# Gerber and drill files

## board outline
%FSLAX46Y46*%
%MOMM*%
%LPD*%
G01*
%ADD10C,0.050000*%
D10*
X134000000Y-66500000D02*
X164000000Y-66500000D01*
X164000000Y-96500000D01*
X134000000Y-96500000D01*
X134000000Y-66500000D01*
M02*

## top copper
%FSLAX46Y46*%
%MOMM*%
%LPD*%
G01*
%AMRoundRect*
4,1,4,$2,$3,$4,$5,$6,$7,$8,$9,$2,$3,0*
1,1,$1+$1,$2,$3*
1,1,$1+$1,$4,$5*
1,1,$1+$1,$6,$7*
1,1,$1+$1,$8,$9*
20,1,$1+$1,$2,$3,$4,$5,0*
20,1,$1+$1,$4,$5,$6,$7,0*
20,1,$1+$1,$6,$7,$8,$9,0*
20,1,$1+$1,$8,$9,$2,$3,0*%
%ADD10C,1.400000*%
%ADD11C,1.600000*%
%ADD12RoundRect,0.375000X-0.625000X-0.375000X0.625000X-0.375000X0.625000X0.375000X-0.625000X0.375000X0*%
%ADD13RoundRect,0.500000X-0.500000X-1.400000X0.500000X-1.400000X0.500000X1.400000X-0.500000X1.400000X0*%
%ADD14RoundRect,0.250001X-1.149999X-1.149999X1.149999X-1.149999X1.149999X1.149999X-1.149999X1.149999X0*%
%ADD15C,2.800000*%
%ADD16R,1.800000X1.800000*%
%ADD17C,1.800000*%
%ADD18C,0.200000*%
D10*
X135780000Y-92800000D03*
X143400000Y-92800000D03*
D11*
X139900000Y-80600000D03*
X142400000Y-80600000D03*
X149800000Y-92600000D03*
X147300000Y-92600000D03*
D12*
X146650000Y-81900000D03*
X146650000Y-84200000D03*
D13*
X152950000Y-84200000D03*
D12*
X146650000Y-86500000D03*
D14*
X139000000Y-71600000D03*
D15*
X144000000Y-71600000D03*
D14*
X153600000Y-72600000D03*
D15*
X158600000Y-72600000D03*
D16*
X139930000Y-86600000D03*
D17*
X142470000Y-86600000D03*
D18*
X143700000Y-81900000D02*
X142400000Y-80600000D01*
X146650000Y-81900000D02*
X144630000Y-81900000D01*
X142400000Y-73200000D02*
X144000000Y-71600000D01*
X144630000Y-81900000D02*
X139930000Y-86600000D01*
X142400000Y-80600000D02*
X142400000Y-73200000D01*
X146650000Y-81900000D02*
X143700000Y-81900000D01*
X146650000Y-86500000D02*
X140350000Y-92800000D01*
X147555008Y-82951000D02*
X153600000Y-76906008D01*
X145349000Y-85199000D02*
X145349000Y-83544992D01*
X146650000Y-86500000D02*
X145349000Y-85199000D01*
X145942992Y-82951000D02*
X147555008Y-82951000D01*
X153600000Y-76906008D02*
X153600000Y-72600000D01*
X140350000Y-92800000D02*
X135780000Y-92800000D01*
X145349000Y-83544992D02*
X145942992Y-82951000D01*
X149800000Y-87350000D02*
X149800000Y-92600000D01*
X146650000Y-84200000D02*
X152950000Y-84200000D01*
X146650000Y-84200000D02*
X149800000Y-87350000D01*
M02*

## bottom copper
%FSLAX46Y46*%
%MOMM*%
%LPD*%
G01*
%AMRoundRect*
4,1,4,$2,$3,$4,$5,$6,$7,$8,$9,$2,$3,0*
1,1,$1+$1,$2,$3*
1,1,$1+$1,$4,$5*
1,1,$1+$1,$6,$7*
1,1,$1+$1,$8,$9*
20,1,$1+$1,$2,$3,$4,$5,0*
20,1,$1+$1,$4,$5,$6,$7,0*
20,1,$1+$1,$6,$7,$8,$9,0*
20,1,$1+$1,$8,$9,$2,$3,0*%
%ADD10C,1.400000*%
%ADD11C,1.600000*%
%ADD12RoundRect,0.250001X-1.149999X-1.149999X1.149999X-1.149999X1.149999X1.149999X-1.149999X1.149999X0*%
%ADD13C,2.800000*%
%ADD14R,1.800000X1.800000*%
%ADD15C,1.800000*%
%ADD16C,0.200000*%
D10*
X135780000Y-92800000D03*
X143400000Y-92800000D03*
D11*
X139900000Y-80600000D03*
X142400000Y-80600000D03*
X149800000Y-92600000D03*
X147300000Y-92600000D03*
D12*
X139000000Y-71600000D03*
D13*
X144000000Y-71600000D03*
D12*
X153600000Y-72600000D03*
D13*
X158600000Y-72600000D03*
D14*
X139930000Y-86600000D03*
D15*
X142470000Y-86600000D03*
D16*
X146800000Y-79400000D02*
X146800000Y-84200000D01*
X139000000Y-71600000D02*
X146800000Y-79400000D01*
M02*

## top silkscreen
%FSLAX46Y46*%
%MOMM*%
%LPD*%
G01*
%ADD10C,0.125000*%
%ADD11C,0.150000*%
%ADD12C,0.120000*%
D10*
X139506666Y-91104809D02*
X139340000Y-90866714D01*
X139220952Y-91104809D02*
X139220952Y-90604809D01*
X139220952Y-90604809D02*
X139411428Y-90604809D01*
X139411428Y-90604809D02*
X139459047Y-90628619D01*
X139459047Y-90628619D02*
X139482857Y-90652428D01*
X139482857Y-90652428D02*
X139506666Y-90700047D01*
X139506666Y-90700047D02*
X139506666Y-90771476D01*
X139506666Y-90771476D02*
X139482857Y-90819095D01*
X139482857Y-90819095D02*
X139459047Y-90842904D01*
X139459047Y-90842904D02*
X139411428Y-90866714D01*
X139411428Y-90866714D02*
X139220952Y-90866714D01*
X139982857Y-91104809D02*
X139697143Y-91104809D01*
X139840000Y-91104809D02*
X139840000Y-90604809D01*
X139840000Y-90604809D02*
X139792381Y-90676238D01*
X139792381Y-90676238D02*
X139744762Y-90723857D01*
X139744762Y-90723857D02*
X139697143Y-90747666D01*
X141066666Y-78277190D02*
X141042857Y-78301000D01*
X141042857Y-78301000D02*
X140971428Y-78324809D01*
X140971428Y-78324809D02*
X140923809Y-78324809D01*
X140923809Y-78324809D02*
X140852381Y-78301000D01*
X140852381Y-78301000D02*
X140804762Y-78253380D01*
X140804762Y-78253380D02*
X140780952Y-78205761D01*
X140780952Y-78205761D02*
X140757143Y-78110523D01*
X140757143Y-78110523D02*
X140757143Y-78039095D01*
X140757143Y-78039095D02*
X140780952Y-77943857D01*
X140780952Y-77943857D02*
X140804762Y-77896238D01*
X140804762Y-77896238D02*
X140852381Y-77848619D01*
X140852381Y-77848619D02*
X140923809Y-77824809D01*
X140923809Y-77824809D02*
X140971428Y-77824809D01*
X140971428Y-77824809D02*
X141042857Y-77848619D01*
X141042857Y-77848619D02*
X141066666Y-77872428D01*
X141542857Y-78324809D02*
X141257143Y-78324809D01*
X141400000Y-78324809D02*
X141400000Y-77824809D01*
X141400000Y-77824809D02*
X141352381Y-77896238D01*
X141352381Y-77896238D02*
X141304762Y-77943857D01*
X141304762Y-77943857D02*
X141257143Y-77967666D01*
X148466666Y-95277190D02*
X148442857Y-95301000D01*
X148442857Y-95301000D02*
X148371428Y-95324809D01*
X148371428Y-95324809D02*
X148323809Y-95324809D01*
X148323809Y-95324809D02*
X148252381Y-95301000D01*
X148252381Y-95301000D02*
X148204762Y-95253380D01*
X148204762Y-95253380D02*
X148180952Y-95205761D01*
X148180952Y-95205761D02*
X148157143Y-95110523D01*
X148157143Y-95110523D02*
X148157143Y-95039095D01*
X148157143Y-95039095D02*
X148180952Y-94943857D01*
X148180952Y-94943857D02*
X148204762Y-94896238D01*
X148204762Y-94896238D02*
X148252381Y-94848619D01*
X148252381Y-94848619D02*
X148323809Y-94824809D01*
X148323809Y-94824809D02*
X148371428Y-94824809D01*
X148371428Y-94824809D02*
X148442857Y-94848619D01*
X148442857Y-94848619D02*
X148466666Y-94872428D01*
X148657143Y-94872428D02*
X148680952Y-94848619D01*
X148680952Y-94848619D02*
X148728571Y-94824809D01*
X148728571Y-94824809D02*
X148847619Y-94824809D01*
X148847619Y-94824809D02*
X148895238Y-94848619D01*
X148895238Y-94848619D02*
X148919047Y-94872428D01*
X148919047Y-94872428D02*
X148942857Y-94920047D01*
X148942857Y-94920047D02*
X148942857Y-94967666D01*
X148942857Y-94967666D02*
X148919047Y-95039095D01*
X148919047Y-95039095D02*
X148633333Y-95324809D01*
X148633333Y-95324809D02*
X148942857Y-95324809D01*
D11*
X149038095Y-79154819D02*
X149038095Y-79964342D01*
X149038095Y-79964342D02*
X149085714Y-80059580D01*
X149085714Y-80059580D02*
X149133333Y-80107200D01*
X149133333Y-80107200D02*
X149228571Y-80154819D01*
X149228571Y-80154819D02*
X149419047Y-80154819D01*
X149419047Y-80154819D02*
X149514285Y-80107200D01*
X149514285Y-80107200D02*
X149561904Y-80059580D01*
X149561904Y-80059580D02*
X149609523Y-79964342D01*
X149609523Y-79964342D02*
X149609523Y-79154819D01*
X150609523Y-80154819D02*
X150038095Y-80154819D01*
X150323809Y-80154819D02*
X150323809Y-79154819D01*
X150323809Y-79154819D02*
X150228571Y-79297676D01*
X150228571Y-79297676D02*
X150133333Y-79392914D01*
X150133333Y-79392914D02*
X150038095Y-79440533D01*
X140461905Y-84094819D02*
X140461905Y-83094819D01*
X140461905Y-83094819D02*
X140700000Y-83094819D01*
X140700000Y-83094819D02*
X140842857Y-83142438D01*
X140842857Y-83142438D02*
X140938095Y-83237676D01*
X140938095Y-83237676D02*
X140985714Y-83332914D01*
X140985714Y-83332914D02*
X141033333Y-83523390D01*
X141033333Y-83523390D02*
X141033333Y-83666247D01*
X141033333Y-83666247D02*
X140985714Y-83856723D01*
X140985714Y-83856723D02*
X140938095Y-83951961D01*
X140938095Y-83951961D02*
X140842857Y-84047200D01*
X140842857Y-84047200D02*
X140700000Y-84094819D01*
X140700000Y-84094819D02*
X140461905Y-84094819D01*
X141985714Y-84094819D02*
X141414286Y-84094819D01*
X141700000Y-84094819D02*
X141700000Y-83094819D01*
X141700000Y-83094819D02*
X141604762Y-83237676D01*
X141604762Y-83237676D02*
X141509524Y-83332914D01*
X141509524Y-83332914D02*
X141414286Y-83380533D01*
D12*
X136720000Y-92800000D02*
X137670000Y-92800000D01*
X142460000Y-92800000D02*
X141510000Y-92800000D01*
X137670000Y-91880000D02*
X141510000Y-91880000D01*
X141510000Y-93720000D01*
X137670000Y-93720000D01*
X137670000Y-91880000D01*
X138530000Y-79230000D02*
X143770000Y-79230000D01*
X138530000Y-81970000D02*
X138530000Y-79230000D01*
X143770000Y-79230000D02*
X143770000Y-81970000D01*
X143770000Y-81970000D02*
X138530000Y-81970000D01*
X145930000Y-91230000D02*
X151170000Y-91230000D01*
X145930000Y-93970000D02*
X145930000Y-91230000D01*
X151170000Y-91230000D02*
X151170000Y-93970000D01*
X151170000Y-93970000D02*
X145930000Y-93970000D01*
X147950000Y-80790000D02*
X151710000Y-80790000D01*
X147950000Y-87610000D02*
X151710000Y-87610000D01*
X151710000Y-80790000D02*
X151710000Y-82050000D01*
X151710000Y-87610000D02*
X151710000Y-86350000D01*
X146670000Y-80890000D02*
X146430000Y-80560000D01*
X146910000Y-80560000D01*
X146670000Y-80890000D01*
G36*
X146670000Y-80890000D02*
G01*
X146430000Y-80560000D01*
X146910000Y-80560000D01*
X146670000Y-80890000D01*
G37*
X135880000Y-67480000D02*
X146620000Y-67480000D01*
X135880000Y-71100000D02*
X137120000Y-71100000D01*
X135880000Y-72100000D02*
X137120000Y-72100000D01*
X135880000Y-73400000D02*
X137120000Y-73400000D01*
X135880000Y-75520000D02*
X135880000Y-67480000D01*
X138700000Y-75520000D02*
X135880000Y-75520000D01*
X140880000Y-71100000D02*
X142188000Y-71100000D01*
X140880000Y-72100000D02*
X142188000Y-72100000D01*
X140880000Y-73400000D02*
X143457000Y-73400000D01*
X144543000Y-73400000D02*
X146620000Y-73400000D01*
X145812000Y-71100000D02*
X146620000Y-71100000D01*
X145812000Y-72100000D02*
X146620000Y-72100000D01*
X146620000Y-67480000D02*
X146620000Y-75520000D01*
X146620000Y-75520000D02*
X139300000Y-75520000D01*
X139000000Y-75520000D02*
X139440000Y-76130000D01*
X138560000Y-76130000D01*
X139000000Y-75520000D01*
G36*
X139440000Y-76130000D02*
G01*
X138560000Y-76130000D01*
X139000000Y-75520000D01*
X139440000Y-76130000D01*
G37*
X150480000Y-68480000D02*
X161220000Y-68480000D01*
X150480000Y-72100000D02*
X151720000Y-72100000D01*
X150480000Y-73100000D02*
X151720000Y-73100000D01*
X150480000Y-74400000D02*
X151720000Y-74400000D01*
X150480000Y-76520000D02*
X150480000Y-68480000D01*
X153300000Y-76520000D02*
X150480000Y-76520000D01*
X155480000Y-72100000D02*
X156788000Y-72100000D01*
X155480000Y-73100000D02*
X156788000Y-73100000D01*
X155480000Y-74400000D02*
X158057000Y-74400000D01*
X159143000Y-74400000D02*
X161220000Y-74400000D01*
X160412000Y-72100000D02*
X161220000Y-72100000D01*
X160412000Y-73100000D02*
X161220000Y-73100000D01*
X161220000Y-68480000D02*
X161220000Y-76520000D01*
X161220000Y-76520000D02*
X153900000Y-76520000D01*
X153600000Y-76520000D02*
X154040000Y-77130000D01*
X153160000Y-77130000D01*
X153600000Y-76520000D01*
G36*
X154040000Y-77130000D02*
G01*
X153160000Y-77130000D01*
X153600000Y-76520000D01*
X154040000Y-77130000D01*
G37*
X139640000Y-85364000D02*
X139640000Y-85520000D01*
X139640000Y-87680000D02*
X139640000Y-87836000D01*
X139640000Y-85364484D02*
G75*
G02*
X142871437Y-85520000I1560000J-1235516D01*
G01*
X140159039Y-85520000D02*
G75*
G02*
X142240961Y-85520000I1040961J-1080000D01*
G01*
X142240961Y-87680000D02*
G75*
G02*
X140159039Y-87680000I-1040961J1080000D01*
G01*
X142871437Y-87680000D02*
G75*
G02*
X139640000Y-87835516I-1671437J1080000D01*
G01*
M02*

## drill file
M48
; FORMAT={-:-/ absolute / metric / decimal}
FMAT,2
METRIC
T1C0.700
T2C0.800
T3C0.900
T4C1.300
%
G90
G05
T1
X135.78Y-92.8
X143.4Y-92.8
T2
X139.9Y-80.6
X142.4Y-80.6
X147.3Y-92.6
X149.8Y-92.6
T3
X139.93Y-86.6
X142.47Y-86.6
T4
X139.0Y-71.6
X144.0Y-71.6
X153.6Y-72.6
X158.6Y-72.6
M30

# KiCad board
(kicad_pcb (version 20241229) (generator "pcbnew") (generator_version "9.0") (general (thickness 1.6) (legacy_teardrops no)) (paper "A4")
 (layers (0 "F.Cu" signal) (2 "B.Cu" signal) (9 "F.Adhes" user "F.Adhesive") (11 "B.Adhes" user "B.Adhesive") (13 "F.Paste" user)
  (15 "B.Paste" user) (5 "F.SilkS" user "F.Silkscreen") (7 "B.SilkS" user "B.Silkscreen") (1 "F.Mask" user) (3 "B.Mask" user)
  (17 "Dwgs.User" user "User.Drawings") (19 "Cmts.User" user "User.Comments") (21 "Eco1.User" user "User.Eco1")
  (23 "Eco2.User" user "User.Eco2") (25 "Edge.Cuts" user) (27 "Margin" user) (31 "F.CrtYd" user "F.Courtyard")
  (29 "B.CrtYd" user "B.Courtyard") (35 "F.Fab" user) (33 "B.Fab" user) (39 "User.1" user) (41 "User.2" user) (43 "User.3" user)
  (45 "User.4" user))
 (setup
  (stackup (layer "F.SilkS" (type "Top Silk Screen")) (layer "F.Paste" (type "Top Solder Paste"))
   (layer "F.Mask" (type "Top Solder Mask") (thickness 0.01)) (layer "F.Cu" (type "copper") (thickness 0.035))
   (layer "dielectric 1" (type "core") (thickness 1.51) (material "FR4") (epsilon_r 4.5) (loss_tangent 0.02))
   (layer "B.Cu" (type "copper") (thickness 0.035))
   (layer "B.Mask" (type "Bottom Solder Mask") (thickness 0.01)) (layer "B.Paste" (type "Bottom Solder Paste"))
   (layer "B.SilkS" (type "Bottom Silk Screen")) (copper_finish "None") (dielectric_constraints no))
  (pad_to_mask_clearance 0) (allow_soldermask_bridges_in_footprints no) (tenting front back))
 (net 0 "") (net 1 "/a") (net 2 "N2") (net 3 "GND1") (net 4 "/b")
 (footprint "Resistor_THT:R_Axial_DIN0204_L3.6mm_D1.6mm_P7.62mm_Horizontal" (layer "F.Cu") (at 135.78 92.8)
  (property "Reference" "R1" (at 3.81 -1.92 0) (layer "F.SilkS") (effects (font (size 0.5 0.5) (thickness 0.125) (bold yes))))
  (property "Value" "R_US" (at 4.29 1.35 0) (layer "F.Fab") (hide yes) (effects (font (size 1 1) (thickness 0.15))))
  (fp_line (start 0.94 0) (end 1.89 0) (stroke (width 0.12) (type solid)) (layer "F.SilkS"))
  (fp_line (start 6.68 0) (end 5.73 0) (stroke (width 0.12) (type solid)) (layer "F.SilkS"))
  (fp_rect (start 1.89 -0.92) (end 5.73 0.92) (stroke (width 0.12) (type solid)) (fill no) (layer "F.SilkS"))
  (pad "1" thru_hole circle (at 0 0) (size 1.4 1.4) (drill 0.7) (layers "*.Cu" "*.Mask") (remove_unused_layers no) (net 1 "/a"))
  (pad "2" thru_hole circle (at 7.62 0) (size 1.4 1.4) (drill 0.7) (layers "*.Cu" "*.Mask") (remove_unused_layers no) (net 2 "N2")))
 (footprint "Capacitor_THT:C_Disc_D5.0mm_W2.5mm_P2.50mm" (layer "F.Cu") (at 139.9 80.6)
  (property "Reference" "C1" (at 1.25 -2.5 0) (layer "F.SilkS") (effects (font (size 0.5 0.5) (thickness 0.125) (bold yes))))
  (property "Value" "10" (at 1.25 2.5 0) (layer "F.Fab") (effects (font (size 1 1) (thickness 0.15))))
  (fp_line (start -1.37 -1.37) (end 3.87 -1.37) (stroke (width 0.12) (type solid)) (layer "F.SilkS"))
  (fp_line (start -1.37 1.37) (end -1.37 -1.37) (stroke (width 0.12) (type solid)) (layer "F.SilkS"))
  (fp_line (start 3.87 -1.37) (end 3.87 1.37) (stroke (width 0.12) (type solid)) (layer "F.SilkS"))
  (fp_line (start 3.87 1.37) (end -1.37 1.37) (stroke (width 0.12) (type solid)) (layer "F.SilkS"))
  (pad "1" thru_hole circle (at 0 0) (size 1.6 1.6) (drill 0.8) (layers "*.Cu" "*.Mask") (remove_unused_layers no) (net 1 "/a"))
  (pad "2" thru_hole circle (at 2.5 0) (size 1.6 1.6) (drill 0.8) (layers "*.Cu" "*.Mask") (remove_unused_layers no) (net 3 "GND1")))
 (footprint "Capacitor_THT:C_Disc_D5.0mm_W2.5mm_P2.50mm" (layer "F.Cu") (at 149.8 92.6 180)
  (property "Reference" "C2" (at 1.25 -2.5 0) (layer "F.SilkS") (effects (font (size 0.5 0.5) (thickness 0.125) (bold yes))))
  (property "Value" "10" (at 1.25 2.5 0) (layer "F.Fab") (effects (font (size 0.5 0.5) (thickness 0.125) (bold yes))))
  (fp_line (start 3.87 1.37) (end -1.37 1.37) (stroke (width 0.12) (type solid)) (layer "F.SilkS"))
  (fp_line (start 3.87 -1.37) (end 3.87 1.37) (stroke (width 0.12) (type solid)) (layer "F.SilkS"))
  (fp_line (start -1.37 1.37) (end -1.37 -1.37) (stroke (width 0.12) (type solid)) (layer "F.SilkS"))
  (fp_line (start -1.37 -1.37) (end 3.87 -1.37) (stroke (width 0.12) (type solid)) (layer "F.SilkS"))
  (pad "1" thru_hole circle (at 0 0 180) (size 1.6 1.6) (drill 0.8) (layers "*.Cu" "*.Mask") (remove_unused_layers no) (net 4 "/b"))
  (pad "2" thru_hole circle (at 2.5 0 180) (size 1.6 1.6) (drill 0.8) (layers "*.Cu" "*.Mask") (remove_unused_layers no) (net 3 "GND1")))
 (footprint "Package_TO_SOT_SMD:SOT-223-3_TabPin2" (layer "F.Cu") (at 149.8 84.2)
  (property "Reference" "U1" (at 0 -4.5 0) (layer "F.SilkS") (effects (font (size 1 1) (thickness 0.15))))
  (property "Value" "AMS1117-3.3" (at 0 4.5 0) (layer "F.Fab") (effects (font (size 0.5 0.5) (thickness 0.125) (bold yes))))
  (fp_line (start -1.85 -3.41) (end 1.91 -3.41) (stroke (width 0.12) (type solid)) (layer "F.SilkS"))
  (fp_line (start -1.85 3.41) (end 1.91 3.41) (stroke (width 0.12) (type solid)) (layer "F.SilkS"))
  (fp_line (start 1.91 -3.41) (end 1.91 -2.15) (stroke (width 0.12) (type solid)) (layer "F.SilkS"))
  (fp_line (start 1.91 3.41) (end 1.91 2.15) (stroke (width 0.12) (type solid)) (layer "F.SilkS"))
  (fp_poly
   (pts (xy -3.13 -3.31) (xy -3.37 -3.64) (xy -2.89 -3.64) (xy -3.13 -3.31)) (stroke (width 0.12) (type solid)) (fill yes) (layer "F.SilkS"))
  (pad "1" smd roundrect (at -3.15 -2.3) (size 2 1.5) (layers "F.Cu" "F.Mask" "F.Paste") (roundrect_rratio 0.25) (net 3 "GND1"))
  (pad "2" smd roundrect (at -3.15 0) (size 2 1.5) (layers "F.Cu" "F.Mask" "F.Paste") (roundrect_rratio 0.25) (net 4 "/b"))
  (pad "2" smd roundrect (at 3.15 0) (size 2 3.8) (layers "F.Cu" "F.Mask" "F.Paste") (roundrect_rratio 0.25) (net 4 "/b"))
  (pad "3" smd roundrect (at -3.15 2.3) (size 2 1.5) (layers "F.Cu" "F.Mask" "F.Paste") (roundrect_rratio 0.25) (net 1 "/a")))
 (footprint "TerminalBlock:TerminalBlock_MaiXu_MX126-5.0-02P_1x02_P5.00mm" (layer "F.Cu") (at 139 71.6)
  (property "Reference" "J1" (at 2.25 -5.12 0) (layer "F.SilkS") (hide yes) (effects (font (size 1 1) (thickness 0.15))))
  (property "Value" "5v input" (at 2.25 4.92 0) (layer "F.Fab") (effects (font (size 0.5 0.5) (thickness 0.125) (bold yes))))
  (fp_line (start -3.12 -4.12) (end 7.62 -4.12) (stroke (width 0.12) (type solid)) (layer "F.SilkS"))
  (fp_line (start -3.12 -0.5) (end -1.88 -0.5) (stroke (width 0.12) (type solid)) (layer "F.SilkS"))
  (fp_line (start -3.12 0.5) (end -1.88 0.5) (stroke (width 0.12) (type solid)) (layer "F.SilkS"))
  (fp_line (start -3.12 1.8) (end -1.88 1.8) (stroke (width 0.12) (type solid)) (layer "F.SilkS"))
  (fp_line (start -3.12 3.92) (end -3.12 -4.12) (stroke (width 0.12) (type solid)) (layer "F.SilkS"))
  (fp_line (start -0.3 3.92) (end -3.12 3.92) (stroke (width 0.12) (type solid)) (layer "F.SilkS"))
  (fp_line (start 1.88 -0.5) (end 3.188 -0.5) (stroke (width 0.12) (type solid)) (layer "F.SilkS"))
  (fp_line (start 1.88 0.5) (end 3.188 0.5) (stroke (width 0.12) (type solid)) (layer "F.SilkS"))
  (fp_line (start 1.88 1.8) (end 4.457 1.8) (stroke (width 0.12) (type solid)) (layer "F.SilkS"))
  (fp_line (start 5.543 1.8) (end 7.62 1.8) (stroke (width 0.12) (type solid)) (layer "F.SilkS"))
  (fp_line (start 6.812 -0.5) (end 7.62 -0.5) (stroke (width 0.12) (type solid)) (layer "F.SilkS"))
  (fp_line (start 6.812 0.5) (end 7.62 0.5) (stroke (width 0.12) (type solid)) (layer "F.SilkS"))
  (fp_line (start 7.62 -4.12) (end 7.62 3.92) (stroke (width 0.12) (type solid)) (layer "F.SilkS"))
  (fp_line (start 7.62 3.92) (end 0.3 3.92) (stroke (width 0.12) (type solid)) (layer "F.SilkS"))
  (fp_poly (pts (xy 0 3.92) (xy 0.44 4.53) (xy -0.44 4.53)) (stroke (width 0.12) (type solid)) (fill yes) (layer "F.SilkS"))
  (pad "1" thru_hole roundrect (at 0 0) (size 2.8 2.8) (drill 1.3) (layers "*.Cu" "*.Mask") (remove_unused_layers no)
   (roundrect_rratio 0.089286) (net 4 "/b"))
  (pad "2" thru_hole circle (at 5 0) (size 2.8 2.8) (drill 1.3) (layers "*.Cu" "*.Mask") (remove_unused_layers no) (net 3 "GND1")))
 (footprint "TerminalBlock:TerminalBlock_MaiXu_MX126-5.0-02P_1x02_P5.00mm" (layer "F.Cu") (at 153.6 72.6)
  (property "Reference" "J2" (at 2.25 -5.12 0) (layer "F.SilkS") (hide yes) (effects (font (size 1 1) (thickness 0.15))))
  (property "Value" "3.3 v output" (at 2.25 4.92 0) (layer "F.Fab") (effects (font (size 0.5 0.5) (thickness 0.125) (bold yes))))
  (fp_line (start -3.12 -4.12) (end 7.62 -4.12) (stroke (width 0.12) (type solid)) (layer "F.SilkS"))
  (fp_line (start -3.12 -0.5) (end -1.88 -0.5) (stroke (width 0.12) (type solid)) (layer "F.SilkS"))
  (fp_line (start -3.12 0.5) (end -1.88 0.5) (stroke (width 0.12) (type solid)) (layer "F.SilkS"))
  (fp_line (start -3.12 1.8) (end -1.88 1.8) (stroke (width 0.12) (type solid)) (layer "F.SilkS"))
  (fp_line (start -3.12 3.92) (end -3.12 -4.12) (stroke (width 0.12) (type solid)) (layer "F.SilkS"))
  (fp_line (start -0.3 3.92) (end -3.12 3.92) (stroke (width 0.12) (type solid)) (layer "F.SilkS"))
  (fp_line (start 1.88 -0.5) (end 3.188 -0.5) (stroke (width 0.12) (type solid)) (layer "F.SilkS"))
  (fp_line (start 1.88 0.5) (end 3.188 0.5) (stroke (width 0.12) (type solid)) (layer "F.SilkS"))
  (fp_line (start 1.88 1.8) (end 4.457 1.8) (stroke (width 0.12) (type solid)) (layer "F.SilkS"))
  (fp_line (start 5.543 1.8) (end 7.62 1.8) (stroke (width 0.12) (type solid)) (layer "F.SilkS"))
  (fp_line (start 6.812 -0.5) (end 7.62 -0.5) (stroke (width 0.12) (type solid)) (layer "F.SilkS"))
  (fp_line (start 6.812 0.5) (end 7.62 0.5) (stroke (width 0.12) (type solid)) (layer "F.SilkS"))
  (fp_line (start 7.62 -4.12) (end 7.62 3.92) (stroke (width 0.12) (type solid)) (layer "F.SilkS"))
  (fp_line (start 7.62 3.92) (end 0.3 3.92) (stroke (width 0.12) (type solid)) (layer "F.SilkS"))
  (fp_poly (pts (xy 0 3.92) (xy 0.44 4.53) (xy -0.44 4.53)) (stroke (width 0.12) (type solid)) (fill yes) (layer "F.SilkS"))
  (pad "1" thru_hole roundrect (at 0 0) (size 2.8 2.8) (drill 1.3) (layers "*.Cu" "*.Mask") (remove_unused_layers no)
   (roundrect_rratio 0.089286) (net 1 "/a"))
  (pad "2" thru_hole circle (at 5 0) (size 2.8 2.8) (drill 1.3) (layers "*.Cu" "*.Mask") (remove_unused_layers no) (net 3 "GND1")))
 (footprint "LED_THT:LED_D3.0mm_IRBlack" (layer "F.Cu") (at 139.93 86.6)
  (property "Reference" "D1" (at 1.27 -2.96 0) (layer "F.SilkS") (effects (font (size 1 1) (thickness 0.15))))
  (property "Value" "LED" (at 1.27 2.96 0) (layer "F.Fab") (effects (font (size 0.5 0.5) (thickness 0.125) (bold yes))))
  (fp_line (start -0.29 -1.236) (end -0.29 -1.08) (stroke (width 0.12) (type solid)) (layer "F.SilkS"))
  (fp_line (start -0.29 1.08) (end -0.29 1.236) (stroke (width 0.12) (type solid)) (layer "F.SilkS"))
  (fp_arc (start -0.29 -1.235516) (mid 1.36566 -1.987699) (end 2.941437 -1.08) (stroke (width 0.12) (type solid)) (layer "F.SilkS"))
  (fp_arc (start 0.229039 -1.08) (mid 1.27 -1.5) (end 2.310961 -1.08) (stroke (width 0.12) (type solid)) (layer "F.SilkS"))
  (fp_arc (start 2.310961 1.08) (mid 1.27 1.5) (end 0.229039 1.08) (stroke (width 0.12) (type solid)) (layer "F.SilkS"))
  (fp_arc (start 2.941437 1.08) (mid 1.36566 1.987699) (end -0.29 1.235516) (stroke (width 0.12) (type solid)) (layer "F.SilkS"))
  (pad "1" thru_hole rect (at 0 0) (size 1.8 1.8) (drill 0.9) (layers "*.Cu" "*.Mask") (remove_unused_layers no) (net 3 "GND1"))
  (pad "2" thru_hole circle (at 2.54 0) (size 1.8 1.8) (drill 0.9) (layers "*.Cu" "*.Mask") (remove_unused_layers no) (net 2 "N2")))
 (gr_rect (start 134 66.5) (end 164 96.5) (stroke (width 0.05) (type default)) (fill no) (layer "Edge.Cuts"))
 (segment (start 143.7 81.9) (end 142.4 80.6) (width 0.2) (layer "F.Cu") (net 3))
 (segment (start 146.65 81.9) (end 144.63 81.9) (width 0.2) (layer "F.Cu") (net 3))
 (segment (start 142.4 73.2) (end 144 71.6) (width 0.2) (layer "F.Cu") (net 3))
 (segment (start 144.63 81.9) (end 139.93 86.6) (width 0.2) (layer "F.Cu") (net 3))
 (segment (start 142.4 80.6) (end 142.4 73.2) (width 0.2) (layer "F.Cu") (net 3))
 (segment (start 146.65 81.9) (end 143.7 81.9) (width 0.2) (layer "F.Cu") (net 3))
 (segment (start 146.65 86.5) (end 140.35 92.8) (width 0.2) (layer "F.Cu") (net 1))
 (segment (start 147.555008 82.951) (end 153.6 76.906008) (width 0.2) (layer "F.Cu") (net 1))
 (segment (start 145.349 85.199) (end 145.349 83.544992) (width 0.2) (layer "F.Cu") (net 1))
 (segment (start 146.65 86.5) (end 145.349 85.199) (width 0.2) (layer "F.Cu") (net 1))
 (segment (start 145.942992 82.951) (end 147.555008 82.951) (width 0.2) (layer "F.Cu") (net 1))
 (segment (start 153.6 76.906008) (end 153.6 72.6) (width 0.2) (layer "F.Cu") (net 1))
 (segment (start 140.35 92.8) (end 135.78 92.8) (width 0.2) (layer "F.Cu") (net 1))
 (segment (start 145.349 83.544992) (end 145.942992 82.951) (width 0.2) (layer "F.Cu") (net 1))
 (segment (start 149.8 87.35) (end 149.8 92.6) (width 0.2) (layer "F.Cu") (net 4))
 (segment (start 146.65 84.2) (end 152.95 84.2) (width 0.2) (layer "F.Cu") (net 4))
 (segment (start 146.65 84.2) (end 149.8 87.35) (width 0.2) (layer "F.Cu") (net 4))
 (segment (start 146.8 79.4) (end 146.8 84.2) (width 0.2) (layer "B.Cu") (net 4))
 (segment (start 139 71.6) (end 146.8 79.4) (width 0.2) (layer "B.Cu") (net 4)))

